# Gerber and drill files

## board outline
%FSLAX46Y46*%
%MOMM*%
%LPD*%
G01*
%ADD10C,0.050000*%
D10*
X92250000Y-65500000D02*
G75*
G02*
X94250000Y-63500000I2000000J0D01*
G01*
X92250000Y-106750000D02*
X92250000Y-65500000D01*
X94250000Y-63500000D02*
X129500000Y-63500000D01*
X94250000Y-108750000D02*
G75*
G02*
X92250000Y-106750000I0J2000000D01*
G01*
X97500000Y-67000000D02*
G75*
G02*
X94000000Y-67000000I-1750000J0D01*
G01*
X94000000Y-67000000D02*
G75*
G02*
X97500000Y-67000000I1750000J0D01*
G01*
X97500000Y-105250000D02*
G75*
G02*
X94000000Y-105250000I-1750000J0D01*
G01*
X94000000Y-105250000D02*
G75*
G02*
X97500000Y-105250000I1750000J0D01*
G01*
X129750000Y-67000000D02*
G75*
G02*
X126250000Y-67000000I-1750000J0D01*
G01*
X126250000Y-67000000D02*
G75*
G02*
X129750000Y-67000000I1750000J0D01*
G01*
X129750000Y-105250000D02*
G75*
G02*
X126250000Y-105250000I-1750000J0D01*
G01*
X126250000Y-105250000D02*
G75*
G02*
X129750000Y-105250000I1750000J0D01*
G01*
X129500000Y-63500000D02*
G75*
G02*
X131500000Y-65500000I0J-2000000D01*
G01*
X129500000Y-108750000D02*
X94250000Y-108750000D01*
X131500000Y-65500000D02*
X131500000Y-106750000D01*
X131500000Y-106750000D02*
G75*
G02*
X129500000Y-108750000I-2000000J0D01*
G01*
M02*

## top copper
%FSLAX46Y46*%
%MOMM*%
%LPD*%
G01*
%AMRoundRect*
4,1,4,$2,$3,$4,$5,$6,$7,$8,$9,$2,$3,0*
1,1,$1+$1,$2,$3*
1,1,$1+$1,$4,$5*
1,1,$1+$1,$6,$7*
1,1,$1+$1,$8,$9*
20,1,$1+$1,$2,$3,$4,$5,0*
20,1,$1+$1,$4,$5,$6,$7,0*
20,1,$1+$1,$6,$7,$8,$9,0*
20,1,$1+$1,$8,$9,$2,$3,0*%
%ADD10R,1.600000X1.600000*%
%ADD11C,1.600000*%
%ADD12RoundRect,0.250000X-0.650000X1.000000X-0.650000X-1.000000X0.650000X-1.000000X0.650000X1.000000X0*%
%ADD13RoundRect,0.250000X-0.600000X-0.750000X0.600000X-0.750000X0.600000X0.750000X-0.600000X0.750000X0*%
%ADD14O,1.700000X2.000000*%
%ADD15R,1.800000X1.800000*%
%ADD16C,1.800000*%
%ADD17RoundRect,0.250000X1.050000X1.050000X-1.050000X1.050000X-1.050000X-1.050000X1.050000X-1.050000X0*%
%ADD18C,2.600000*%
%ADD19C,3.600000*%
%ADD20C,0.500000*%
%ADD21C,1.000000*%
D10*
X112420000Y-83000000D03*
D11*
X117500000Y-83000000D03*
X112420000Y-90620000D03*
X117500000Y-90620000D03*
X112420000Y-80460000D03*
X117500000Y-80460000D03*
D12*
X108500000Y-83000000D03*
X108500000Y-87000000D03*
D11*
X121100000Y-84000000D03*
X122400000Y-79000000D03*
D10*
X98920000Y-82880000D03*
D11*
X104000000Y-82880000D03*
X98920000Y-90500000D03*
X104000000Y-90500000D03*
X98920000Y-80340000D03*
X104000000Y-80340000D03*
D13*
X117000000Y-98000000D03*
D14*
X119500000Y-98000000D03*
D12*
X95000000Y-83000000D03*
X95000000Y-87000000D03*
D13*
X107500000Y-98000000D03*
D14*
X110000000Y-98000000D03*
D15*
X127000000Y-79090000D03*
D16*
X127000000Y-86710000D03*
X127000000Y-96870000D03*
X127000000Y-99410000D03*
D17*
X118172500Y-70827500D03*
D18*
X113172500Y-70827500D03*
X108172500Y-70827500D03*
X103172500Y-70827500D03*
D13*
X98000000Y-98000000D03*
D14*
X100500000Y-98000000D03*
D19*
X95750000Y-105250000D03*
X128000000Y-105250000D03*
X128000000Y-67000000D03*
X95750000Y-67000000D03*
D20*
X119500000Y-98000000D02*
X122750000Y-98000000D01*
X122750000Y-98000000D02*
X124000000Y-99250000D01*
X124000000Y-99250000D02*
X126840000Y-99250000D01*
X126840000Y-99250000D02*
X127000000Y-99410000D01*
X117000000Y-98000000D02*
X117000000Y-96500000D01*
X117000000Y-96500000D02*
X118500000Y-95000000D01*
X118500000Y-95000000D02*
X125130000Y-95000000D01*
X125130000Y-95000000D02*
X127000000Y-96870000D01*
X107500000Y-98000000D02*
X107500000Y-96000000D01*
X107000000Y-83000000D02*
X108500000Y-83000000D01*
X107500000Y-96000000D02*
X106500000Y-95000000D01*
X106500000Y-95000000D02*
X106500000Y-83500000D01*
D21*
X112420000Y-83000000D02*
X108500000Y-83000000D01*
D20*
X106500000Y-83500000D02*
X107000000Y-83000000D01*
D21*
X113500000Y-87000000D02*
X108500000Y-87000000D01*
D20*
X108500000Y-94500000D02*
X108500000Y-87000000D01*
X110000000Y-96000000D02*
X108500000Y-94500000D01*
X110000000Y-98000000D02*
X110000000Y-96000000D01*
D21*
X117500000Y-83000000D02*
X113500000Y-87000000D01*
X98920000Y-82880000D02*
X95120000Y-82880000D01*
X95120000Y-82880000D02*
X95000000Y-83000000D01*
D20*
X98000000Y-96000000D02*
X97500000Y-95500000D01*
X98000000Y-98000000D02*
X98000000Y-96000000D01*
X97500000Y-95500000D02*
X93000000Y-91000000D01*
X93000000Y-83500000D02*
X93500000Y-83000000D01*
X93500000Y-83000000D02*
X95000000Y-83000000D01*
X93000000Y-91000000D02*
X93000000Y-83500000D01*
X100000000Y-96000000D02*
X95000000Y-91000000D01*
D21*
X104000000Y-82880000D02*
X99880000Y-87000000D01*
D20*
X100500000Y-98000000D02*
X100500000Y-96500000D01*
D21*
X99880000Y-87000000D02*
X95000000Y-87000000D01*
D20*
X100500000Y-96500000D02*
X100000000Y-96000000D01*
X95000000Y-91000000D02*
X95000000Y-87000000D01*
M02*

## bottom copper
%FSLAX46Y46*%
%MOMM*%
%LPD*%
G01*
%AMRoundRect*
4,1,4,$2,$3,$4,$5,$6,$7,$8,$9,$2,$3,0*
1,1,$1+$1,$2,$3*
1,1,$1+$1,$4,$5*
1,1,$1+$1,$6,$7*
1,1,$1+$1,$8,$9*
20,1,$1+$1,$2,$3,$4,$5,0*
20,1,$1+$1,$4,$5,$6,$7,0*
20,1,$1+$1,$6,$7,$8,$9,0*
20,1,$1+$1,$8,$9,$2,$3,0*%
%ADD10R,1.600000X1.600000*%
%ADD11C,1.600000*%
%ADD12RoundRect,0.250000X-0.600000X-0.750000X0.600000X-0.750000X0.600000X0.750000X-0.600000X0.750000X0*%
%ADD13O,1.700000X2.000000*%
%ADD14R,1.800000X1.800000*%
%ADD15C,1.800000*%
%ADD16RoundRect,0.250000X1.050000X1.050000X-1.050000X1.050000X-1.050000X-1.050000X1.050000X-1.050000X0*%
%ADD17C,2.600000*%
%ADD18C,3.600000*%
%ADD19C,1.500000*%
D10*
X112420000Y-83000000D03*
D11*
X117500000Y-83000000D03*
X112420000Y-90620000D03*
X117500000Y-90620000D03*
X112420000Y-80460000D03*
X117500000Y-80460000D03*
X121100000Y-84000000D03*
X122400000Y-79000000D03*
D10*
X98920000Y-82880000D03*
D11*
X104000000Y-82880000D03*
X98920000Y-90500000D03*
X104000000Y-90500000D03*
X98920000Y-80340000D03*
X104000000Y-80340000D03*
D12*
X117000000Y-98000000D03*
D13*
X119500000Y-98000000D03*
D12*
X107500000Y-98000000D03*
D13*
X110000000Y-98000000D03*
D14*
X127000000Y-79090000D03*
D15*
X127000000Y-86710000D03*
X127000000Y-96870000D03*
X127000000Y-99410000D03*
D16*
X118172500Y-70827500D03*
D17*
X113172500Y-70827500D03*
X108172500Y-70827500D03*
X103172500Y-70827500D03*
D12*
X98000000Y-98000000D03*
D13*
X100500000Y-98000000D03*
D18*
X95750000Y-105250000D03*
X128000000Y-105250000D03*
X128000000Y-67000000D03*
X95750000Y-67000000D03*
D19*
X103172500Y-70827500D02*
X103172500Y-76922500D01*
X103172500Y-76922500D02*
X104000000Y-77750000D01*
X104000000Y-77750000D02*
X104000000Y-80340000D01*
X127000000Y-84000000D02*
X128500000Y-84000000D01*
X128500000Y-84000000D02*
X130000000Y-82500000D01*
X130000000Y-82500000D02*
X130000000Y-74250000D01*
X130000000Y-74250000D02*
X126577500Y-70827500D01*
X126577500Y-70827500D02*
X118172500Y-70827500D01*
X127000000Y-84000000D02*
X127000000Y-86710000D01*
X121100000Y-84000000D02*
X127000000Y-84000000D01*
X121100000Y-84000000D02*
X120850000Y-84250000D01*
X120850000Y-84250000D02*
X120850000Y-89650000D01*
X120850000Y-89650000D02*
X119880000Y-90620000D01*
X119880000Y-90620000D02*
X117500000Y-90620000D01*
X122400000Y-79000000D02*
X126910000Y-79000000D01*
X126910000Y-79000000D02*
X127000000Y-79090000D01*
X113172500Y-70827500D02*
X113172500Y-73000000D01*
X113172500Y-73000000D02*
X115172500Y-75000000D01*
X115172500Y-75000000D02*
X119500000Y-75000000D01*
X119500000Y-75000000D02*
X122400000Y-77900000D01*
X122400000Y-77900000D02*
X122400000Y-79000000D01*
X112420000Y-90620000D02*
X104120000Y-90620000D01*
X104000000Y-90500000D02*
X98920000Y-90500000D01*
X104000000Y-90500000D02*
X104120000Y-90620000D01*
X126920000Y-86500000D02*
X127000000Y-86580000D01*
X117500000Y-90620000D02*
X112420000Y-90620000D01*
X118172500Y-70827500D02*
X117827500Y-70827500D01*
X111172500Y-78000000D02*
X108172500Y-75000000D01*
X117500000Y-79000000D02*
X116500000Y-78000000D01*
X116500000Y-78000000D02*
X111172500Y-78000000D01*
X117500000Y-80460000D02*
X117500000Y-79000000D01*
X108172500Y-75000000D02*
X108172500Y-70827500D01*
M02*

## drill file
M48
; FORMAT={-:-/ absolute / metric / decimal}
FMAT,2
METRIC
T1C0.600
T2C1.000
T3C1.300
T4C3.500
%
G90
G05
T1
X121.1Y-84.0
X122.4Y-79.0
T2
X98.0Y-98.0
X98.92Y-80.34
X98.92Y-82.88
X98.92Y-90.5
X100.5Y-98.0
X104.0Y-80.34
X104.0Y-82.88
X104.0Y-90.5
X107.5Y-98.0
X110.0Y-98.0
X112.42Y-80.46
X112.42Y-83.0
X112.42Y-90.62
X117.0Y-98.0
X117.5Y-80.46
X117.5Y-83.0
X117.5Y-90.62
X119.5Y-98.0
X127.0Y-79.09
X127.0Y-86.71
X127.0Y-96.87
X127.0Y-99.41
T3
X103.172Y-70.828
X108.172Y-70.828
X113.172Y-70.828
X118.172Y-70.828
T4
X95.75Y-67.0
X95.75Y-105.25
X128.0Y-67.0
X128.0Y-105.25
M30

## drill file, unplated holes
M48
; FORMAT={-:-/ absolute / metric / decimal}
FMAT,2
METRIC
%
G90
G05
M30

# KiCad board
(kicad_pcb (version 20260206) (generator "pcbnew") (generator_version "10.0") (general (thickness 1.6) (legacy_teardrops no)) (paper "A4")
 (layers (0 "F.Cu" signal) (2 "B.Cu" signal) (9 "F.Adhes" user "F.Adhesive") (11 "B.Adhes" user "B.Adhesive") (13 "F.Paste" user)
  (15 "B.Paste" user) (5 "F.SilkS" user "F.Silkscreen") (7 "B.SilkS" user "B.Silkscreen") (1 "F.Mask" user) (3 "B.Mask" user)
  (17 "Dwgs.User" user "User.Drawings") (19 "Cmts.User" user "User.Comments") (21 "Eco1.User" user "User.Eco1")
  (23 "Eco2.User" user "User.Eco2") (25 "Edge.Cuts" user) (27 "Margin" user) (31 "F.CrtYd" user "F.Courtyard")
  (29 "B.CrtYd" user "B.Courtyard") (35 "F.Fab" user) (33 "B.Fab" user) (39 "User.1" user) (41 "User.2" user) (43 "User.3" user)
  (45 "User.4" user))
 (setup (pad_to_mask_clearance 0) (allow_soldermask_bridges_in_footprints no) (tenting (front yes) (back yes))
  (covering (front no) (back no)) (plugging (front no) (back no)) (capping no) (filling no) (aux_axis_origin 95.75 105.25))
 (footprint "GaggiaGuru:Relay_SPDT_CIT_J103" (layer "F.Cu") (at 112.42 83 90)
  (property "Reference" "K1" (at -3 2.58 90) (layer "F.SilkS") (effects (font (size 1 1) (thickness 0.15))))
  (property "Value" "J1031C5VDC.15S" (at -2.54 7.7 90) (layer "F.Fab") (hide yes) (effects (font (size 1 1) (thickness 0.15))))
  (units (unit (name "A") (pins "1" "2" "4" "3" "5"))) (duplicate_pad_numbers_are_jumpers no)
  (pad "1" thru_hole rect (at 0 0 90) (size 1.6 1.6) (drill 1) (layers "*.Cu" "*.Mask") (remove_unused_layers no) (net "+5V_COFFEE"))
  (pad "2" thru_hole circle (at 0 5.08 90) (size 1.6 1.6) (drill 1) (layers "*.Cu" "*.Mask") (remove_unused_layers no)
   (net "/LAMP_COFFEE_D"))
  (pad "3" thru_hole circle (at -7.62 0 90) (size 1.6 1.6) (drill 1) (layers "*.Cu" "*.Mask") (remove_unused_layers no) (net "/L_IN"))
  (pad "3" thru_hole circle (at -7.62 5.08 90) (size 1.6 1.6) (drill 1) (layers "*.Cu" "*.Mask") (remove_unused_layers no) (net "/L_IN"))
  (pad "4" thru_hole circle (at 2.54 0 90) (size 1.6 1.6) (drill 1) (layers "*.Cu" "*.Mask") (remove_unused_layers no)
   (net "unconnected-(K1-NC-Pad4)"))
  (pad "5" thru_hole circle (at 2.54 5.08 90) (size 1.6 1.6) (drill 1) (layers "*.Cu" "*.Mask") (remove_unused_layers no)
   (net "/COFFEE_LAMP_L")))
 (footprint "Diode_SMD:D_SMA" (layer "F.Cu") (at 108.5 85 -90)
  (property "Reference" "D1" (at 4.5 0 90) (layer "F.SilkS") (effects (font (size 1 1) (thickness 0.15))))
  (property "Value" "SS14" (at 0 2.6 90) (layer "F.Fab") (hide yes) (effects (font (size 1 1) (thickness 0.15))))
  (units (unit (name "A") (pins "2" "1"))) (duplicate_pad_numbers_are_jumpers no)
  (pad "1" smd roundrect (at -2 0 270) (size 2.5 1.8) (layers "F.Cu" "F.Mask" "F.Paste") (roundrect_rratio 0.1388888889) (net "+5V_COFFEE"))
  (pad "2" smd roundrect (at 2 0 270) (size 2.5 1.8) (layers "F.Cu" "F.Mask" "F.Paste") (roundrect_rratio 0.1388888889)
   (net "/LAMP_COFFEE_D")))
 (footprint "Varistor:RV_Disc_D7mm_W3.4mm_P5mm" (layer "F.Cu") (at 121.1 84 90)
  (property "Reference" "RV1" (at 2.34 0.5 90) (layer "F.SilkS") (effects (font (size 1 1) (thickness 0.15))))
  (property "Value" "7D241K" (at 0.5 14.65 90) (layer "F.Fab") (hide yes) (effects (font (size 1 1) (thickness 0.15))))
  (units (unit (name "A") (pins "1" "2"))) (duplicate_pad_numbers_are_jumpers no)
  (pad "1" thru_hole circle (at 0 0 90) (size 1.6 1.6) (drill 0.6) (layers "*.Cu" "*.Mask") (remove_unused_layers no) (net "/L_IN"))
  (pad "2" thru_hole circle (at 5 1.3 90) (size 1.6 1.6) (drill 0.6) (layers "*.Cu" "*.Mask") (remove_unused_layers no) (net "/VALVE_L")))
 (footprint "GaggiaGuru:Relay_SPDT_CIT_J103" (layer "F.Cu") (at 98.92 82.88 90)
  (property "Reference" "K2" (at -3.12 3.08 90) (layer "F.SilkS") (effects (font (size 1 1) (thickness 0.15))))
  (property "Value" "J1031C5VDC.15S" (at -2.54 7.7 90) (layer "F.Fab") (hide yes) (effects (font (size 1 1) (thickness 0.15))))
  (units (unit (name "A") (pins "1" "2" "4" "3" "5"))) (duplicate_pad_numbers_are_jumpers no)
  (pad "1" thru_hole rect (at 0 0 90) (size 1.6 1.6) (drill 1) (layers "*.Cu" "*.Mask") (remove_unused_layers no) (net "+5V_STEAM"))
  (pad "2" thru_hole circle (at 0 5.08 90) (size 1.6 1.6) (drill 1) (layers "*.Cu" "*.Mask") (remove_unused_layers no) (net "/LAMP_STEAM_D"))
  (pad "3" thru_hole circle (at -7.62 0 90) (size 1.6 1.6) (drill 1) (layers "*.Cu" "*.Mask") (remove_unused_layers no) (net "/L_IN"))
  (pad "3" thru_hole circle (at -7.62 5.08 90) (size 1.6 1.6) (drill 1) (layers "*.Cu" "*.Mask") (remove_unused_layers no) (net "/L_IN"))
  (pad "4" thru_hole circle (at 2.54 0 90) (size 1.6 1.6) (drill 1) (layers "*.Cu" "*.Mask") (remove_unused_layers no)
   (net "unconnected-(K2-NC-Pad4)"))
  (pad "5" thru_hole circle (at 2.54 5.08 90) (size 1.6 1.6) (drill 1) (layers "*.Cu" "*.Mask") (remove_unused_layers no)
   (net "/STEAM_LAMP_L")))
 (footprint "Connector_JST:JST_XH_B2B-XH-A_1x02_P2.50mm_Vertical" (layer "F.Cu") (at 117 98)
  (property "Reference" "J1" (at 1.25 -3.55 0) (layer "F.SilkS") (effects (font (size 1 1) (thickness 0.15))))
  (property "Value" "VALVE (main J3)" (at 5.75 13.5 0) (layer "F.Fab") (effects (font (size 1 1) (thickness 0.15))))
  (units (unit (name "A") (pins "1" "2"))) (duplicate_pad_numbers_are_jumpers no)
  (pad "1" thru_hole roundrect (at 0 0) (size 1.7 2) (drill 1) (layers "*.Cu" "*.Mask") (remove_unused_layers no)
   (roundrect_rratio 0.147059) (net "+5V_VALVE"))
  (pad "2" thru_hole oval (at 2.5 0) (size 1.7 2) (drill 1) (layers "*.Cu" "*.Mask") (remove_unused_layers no) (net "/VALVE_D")))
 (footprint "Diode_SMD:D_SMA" (layer "F.Cu") (at 95 85 -90)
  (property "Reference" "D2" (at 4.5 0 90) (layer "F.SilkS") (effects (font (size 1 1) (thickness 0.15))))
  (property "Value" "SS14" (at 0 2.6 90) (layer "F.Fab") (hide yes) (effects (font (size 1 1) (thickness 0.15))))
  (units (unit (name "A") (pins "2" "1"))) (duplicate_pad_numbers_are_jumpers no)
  (pad "1" smd roundrect (at -2 0 270) (size 2.5 1.8) (layers "F.Cu" "F.Mask" "F.Paste") (roundrect_rratio 0.1388888889) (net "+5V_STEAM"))
  (pad "2" smd roundrect (at 2 0 270) (size 2.5 1.8) (layers "F.Cu" "F.Mask" "F.Paste") (roundrect_rratio 0.1388888889)
   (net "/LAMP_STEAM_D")))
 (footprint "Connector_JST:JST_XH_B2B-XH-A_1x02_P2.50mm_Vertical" (layer "F.Cu") (at 107.5 98)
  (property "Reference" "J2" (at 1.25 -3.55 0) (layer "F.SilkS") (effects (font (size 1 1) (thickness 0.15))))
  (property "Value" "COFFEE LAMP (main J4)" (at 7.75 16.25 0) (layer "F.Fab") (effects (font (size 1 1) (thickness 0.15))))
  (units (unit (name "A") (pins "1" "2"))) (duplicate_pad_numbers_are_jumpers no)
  (pad "1" thru_hole roundrect (at 0 0) (size 1.7 2) (drill 1) (layers "*.Cu" "*.Mask") (remove_unused_layers no)
   (roundrect_rratio 0.147059) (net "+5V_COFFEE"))
  (pad "2" thru_hole oval (at 2.5 0) (size 1.7 2) (drill 1) (layers "*.Cu" "*.Mask") (remove_unused_layers no) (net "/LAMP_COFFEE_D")))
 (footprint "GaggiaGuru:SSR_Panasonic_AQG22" (layer "F.Cu") (at 127 79.09 -90)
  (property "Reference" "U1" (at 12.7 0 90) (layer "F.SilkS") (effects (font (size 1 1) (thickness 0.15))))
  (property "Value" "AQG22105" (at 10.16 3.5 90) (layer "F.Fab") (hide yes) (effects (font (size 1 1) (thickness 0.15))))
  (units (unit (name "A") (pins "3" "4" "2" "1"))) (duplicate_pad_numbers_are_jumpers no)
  (pad "1" thru_hole rect (at 0 0 270) (size 1.8 1.8) (drill 1) (layers "*.Cu" "*.Mask") (remove_unused_layers no) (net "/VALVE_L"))
  (pad "2" thru_hole circle (at 7.62 0 270) (size 1.8 1.8) (drill 1) (layers "*.Cu" "*.Mask") (remove_unused_layers no) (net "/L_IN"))
  (pad "3" thru_hole circle (at 17.78 0 270) (size 1.8 1.8) (drill 1) (layers "*.Cu" "*.Mask") (remove_unused_layers no) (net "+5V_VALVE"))
  (pad "4" thru_hole circle (at 20.32 0 270) (size 1.8 1.8) (drill 1) (layers "*.Cu" "*.Mask") (remove_unused_layers no) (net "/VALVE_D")))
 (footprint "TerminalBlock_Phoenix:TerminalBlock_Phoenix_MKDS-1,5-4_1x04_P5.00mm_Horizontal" (layer "F.Cu") (at 118.1725 70.8275 180)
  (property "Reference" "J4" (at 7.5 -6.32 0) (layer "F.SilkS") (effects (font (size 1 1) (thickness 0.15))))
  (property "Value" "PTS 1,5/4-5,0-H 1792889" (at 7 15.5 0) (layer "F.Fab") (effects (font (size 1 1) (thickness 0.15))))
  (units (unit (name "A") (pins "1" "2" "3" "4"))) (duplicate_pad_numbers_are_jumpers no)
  (pad "1" thru_hole roundrect (at 0 0 180) (size 2.6 2.6) (drill 1.3) (layers "*.Cu" "*.Mask") (remove_unused_layers no)
   (roundrect_rratio 0.096154) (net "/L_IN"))
  (pad "2" thru_hole circle (at 5 0 180) (size 2.6 2.6) (drill 1.3) (layers "*.Cu" "*.Mask") (remove_unused_layers no) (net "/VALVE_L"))
  (pad "3" thru_hole circle (at 10 0 180) (size 2.6 2.6) (drill 1.3) (layers "*.Cu" "*.Mask") (remove_unused_layers no)
   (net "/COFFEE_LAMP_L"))
  (pad "4" thru_hole circle (at 15 0 180) (size 2.6 2.6) (drill 1.3) (layers "*.Cu" "*.Mask") (remove_unused_layers no)
   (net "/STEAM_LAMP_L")))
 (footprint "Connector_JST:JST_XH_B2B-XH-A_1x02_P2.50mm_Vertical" (layer "F.Cu") (at 98 98)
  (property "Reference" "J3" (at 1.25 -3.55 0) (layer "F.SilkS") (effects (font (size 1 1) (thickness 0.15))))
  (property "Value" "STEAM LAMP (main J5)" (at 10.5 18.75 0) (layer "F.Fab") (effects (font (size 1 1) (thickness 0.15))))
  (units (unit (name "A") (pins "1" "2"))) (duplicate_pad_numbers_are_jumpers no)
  (pad "1" thru_hole roundrect (at 0 0) (size 1.7 2) (drill 1) (layers "*.Cu" "*.Mask") (remove_unused_layers no)
   (roundrect_rratio 0.147059) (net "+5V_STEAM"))
  (pad "2" thru_hole oval (at 2.5 0) (size 1.7 2) (drill 1) (layers "*.Cu" "*.Mask") (remove_unused_layers no) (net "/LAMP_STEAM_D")))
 (gr_arc (start 92.25 65.5) (mid 92.835786 64.085786) (end 94.25 63.5) (stroke (width 0.05) (type default)) (layer "Edge.Cuts"))
 (gr_line (start 92.25 106.75) (end 92.25 65.5) (stroke (width 0.05) (type default)) (layer "Edge.Cuts"))
 (gr_line (start 94.25 63.5) (end 129.5 63.5) (stroke (width 0.05) (type default)) (layer "Edge.Cuts"))
 (gr_arc (start 94.25 108.75) (mid 92.835786 108.164214) (end 92.25 106.75) (stroke (width 0.05) (type default)) (layer "Edge.Cuts"))
 (gr_circle (center 95.75 67) (end 97.5 67) (stroke (width 0.05) (type solid)) (fill no) (layer "Edge.Cuts"))
 (gr_circle (center 95.75 105.25) (end 97.5 105.25) (stroke (width 0.05) (type solid)) (fill no) (layer "Edge.Cuts"))
 (gr_circle (center 128 67) (end 129.75 67) (stroke (width 0.05) (type solid)) (fill no) (layer "Edge.Cuts"))
 (gr_circle (center 128 105.25) (end 129.75 105.25) (stroke (width 0.05) (type solid)) (fill no) (layer "Edge.Cuts"))
 (gr_arc (start 129.5 63.5) (mid 130.914214 64.085786) (end 131.5 65.5) (stroke (width 0.05) (type default)) (layer "Edge.Cuts"))
 (gr_line (start 129.5 108.75) (end 94.25 108.75) (stroke (width 0.05) (type default)) (layer "Edge.Cuts"))
 (gr_line (start 131.5 65.5) (end 131.5 106.75) (stroke (width 0.05) (type default)) (layer "Edge.Cuts"))
 (gr_arc (start 131.5 106.75) (mid 130.914214 108.164214) (end 129.5 108.75) (stroke (width 0.05) (type default)) (layer "Edge.Cuts"))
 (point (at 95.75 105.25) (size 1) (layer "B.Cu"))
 (via (at 95.75 105.25) (size 3.6) (drill 3.5) (layers "F.Cu" "B.Cu") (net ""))
 (via (at 128 67) (size 3.6) (drill 3.5) (layers "F.Cu" "B.Cu") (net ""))
 (via (at 128 105.25) (size 3.6) (drill 3.5) (layers "F.Cu" "B.Cu") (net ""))
 (via (at 95.75 67) (size 3.6) (drill 3.5) (layers "F.Cu" "B.Cu") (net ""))
 (segment (start 107.5 98) (end 107.5 96) (width 0.5) (layer "F.Cu") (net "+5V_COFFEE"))
 (segment (start 107 83) (end 108.5 83) (width 0.5) (layer "F.Cu") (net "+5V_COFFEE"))
 (segment (start 107.5 96) (end 106.5 95) (width 0.5) (layer "F.Cu") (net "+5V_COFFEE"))
 (segment (start 106.5 95) (end 106.5 83.5) (width 0.5) (layer "F.Cu") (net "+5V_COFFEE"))
 (segment (start 112.42 83) (end 108.5 83) (width 1) (layer "F.Cu") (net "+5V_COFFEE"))
 (segment (start 106.5 83.5) (end 107 83) (width 0.5) (layer "F.Cu") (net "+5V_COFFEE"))
 (segment (start 113.5 87) (end 108.5 87) (width 1) (layer "F.Cu") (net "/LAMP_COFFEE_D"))
 (segment (start 108.5 94.5) (end 108.5 87) (width 0.5) (layer "F.Cu") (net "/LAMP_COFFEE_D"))
 (segment (start 110 96) (end 108.5 94.5) (width 0.5) (layer "F.Cu") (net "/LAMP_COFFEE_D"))
 (segment (start 110 98) (end 110 96) (width 0.5) (layer "F.Cu") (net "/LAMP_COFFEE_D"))
 (segment (start 117.5 83) (end 113.5 87) (width 1) (layer "F.Cu") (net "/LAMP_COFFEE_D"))
 (segment (start 112.42 90.62) (end 104.12 90.62) (width 1.5) (layer "B.Cu") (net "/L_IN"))
 (segment (start 104 90.5) (end 98.92 90.5) (width 1.5) (layer "B.Cu") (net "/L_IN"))
 (segment (start 104 90.5) (end 104.12 90.62) (width 1.5) (layer "B.Cu") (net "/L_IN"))
 (segment (start 119.88 90.62) (end 117.5 90.62) (width 1.5) (layer "B.Cu") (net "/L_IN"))
 (segment (start 130 82.5) (end 130 74.25) (width 1.5) (layer "B.Cu") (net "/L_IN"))
 (segment (start 127 84) (end 128.5 84) (width 1.5) (layer "B.Cu") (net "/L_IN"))
 (segment (start 120.85 89.65) (end 119.88 90.62) (width 1.5) (layer "B.Cu") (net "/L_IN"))
 (segment (start 127 84) (end 127 86.71) (width 1.5) (layer "B.Cu") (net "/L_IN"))
 (segment (start 126.92 86.5) (end 127 86.58) (width 1.5) (layer "B.Cu") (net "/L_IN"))
 (segment (start 130 74.25) (end 126.5775 70.8275) (width 1.5) (layer "B.Cu") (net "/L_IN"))
 (segment (start 128.5 84) (end 130 82.5) (width 1.5) (layer "B.Cu") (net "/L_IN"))
 (segment (start 126.5775 70.8275) (end 118.1725 70.8275) (width 1.5) (layer "B.Cu") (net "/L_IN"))
 (segment (start 117.5 90.62) (end 112.42 90.62) (width 1.5) (layer "B.Cu") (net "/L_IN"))
 (segment (start 118.1725 70.8275) (end 117.8275 70.8275) (width 1.5) (layer "B.Cu") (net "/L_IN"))
 (segment (start 121.1 84) (end 120.85 84.25) (width 1.5) (layer "B.Cu") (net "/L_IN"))
 (segment (start 120.85 84.25) (end 120.85 89.65) (width 1.5) (layer "B.Cu") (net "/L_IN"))
 (segment (start 121.1 84) (end 127 84) (width 1.5) (layer "B.Cu") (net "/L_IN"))
 (segment (start 111.1725 78) (end 108.1725 75) (width 1.5) (layer "B.Cu") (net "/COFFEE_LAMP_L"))
 (segment (start 117.5 79) (end 116.5 78) (width 1.5) (layer "B.Cu") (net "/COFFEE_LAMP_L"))
 (segment (start 116.5 78) (end 111.1725 78) (width 1.5) (layer "B.Cu") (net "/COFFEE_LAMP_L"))
 (segment (start 117.5 80.46) (end 117.5 79) (width 1.5) (layer "B.Cu") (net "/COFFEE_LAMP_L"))
 (segment (start 108.1725 75) (end 108.1725 70.8275) (width 1.5) (layer "B.Cu") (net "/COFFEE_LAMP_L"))
 (segment (start 119.5 75) (end 122.4 77.9) (width 1.5) (layer "B.Cu") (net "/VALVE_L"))
 (segment (start 122.4 77.9) (end 122.4 79) (width 1.5) (layer "B.Cu") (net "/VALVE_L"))
 (segment (start 122.4 79) (end 126.91 79) (width 1.5) (layer "B.Cu") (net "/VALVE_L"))
 (segment (start 113.1725 73) (end 115.1725 75) (width 1.5) (layer "B.Cu") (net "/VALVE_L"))
 (segment (start 113.1725 70.8275) (end 113.1725 73) (width 1.5) (layer "B.Cu") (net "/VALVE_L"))
 (segment (start 126.91 79) (end 127 79.09) (width 1.5) (layer "B.Cu") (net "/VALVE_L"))
 (segment (start 115.1725 75) (end 119.5 75) (width 1.5) (layer "B.Cu") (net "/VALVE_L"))
 (segment (start 98.92 82.88) (end 95.12 82.88) (width 1) (layer "F.Cu") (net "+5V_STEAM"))
 (segment (start 95.12 82.88) (end 95 83) (width 1) (layer "F.Cu") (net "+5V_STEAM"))
 (segment (start 98 96) (end 97.5 95.5) (width 0.5) (layer "F.Cu") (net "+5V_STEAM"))
 (segment (start 98 98) (end 98 96) (width 0.5) (layer "F.Cu") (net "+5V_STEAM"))
 (segment (start 97.5 95.5) (end 93 91) (width 0.5) (layer "F.Cu") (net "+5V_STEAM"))
 (segment (start 93 83.5) (end 93.5 83) (width 0.5) (layer "F.Cu") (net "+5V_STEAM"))
 (segment (start 93.5 83) (end 95 83) (width 0.5) (layer "F.Cu") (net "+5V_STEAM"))
 (segment (start 93 91) (end 93 83.5) (width 0.5) (layer "F.Cu") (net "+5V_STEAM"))
 (segment (start 100 96) (end 95 91) (width 0.5) (layer "F.Cu") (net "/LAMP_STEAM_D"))
 (segment (start 104 82.88) (end 99.88 87) (width 1) (layer "F.Cu") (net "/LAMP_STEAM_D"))
 (segment (start 100.5 98) (end 100.5 96.5) (width 0.5) (layer "F.Cu") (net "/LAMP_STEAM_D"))
 (segment (start 99.88 87) (end 95 87) (width 1) (layer "F.Cu") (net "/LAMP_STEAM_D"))
 (segment (start 100.5 96.5) (end 100 96) (width 0.5) (layer "F.Cu") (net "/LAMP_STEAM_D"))
 (segment (start 95 91) (end 95 87) (width 0.5) (layer "F.Cu") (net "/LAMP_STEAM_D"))
 (segment (start 103.1725 70.8275) (end 103.1725 76.9225) (width 1.5) (layer "B.Cu") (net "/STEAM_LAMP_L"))
 (segment (start 103.1725 76.9225) (end 104 77.75) (width 1.5) (layer "B.Cu") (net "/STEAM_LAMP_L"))
 (segment (start 104 77.75) (end 104 80.34) (width 1.5) (layer "B.Cu") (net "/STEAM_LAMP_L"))
 (segment (start 117 96.5) (end 118.5 95) (width 0.5) (layer "F.Cu") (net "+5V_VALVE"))
 (segment (start 118.5 95) (end 125.13 95) (width 0.5) (layer "F.Cu") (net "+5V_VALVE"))
 (segment (start 125.13 95) (end 127 96.87) (width 0.5) (layer "F.Cu") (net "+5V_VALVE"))
 (segment (start 117 98) (end 117 96.5) (width 0.5) (layer "F.Cu") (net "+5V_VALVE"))
 (segment (start 122.75 98) (end 124 99.25) (width 0.5) (layer "F.Cu") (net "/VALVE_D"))
 (segment (start 124 99.25) (end 126.84 99.25) (width 0.5) (layer "F.Cu") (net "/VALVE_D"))
 (segment (start 119.5 98) (end 122.75 98) (width 0.5) (layer "F.Cu") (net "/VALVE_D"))
 (segment (start 126.84 99.25) (end 127 99.41) (width 0.5) (layer "F.Cu") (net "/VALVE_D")))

